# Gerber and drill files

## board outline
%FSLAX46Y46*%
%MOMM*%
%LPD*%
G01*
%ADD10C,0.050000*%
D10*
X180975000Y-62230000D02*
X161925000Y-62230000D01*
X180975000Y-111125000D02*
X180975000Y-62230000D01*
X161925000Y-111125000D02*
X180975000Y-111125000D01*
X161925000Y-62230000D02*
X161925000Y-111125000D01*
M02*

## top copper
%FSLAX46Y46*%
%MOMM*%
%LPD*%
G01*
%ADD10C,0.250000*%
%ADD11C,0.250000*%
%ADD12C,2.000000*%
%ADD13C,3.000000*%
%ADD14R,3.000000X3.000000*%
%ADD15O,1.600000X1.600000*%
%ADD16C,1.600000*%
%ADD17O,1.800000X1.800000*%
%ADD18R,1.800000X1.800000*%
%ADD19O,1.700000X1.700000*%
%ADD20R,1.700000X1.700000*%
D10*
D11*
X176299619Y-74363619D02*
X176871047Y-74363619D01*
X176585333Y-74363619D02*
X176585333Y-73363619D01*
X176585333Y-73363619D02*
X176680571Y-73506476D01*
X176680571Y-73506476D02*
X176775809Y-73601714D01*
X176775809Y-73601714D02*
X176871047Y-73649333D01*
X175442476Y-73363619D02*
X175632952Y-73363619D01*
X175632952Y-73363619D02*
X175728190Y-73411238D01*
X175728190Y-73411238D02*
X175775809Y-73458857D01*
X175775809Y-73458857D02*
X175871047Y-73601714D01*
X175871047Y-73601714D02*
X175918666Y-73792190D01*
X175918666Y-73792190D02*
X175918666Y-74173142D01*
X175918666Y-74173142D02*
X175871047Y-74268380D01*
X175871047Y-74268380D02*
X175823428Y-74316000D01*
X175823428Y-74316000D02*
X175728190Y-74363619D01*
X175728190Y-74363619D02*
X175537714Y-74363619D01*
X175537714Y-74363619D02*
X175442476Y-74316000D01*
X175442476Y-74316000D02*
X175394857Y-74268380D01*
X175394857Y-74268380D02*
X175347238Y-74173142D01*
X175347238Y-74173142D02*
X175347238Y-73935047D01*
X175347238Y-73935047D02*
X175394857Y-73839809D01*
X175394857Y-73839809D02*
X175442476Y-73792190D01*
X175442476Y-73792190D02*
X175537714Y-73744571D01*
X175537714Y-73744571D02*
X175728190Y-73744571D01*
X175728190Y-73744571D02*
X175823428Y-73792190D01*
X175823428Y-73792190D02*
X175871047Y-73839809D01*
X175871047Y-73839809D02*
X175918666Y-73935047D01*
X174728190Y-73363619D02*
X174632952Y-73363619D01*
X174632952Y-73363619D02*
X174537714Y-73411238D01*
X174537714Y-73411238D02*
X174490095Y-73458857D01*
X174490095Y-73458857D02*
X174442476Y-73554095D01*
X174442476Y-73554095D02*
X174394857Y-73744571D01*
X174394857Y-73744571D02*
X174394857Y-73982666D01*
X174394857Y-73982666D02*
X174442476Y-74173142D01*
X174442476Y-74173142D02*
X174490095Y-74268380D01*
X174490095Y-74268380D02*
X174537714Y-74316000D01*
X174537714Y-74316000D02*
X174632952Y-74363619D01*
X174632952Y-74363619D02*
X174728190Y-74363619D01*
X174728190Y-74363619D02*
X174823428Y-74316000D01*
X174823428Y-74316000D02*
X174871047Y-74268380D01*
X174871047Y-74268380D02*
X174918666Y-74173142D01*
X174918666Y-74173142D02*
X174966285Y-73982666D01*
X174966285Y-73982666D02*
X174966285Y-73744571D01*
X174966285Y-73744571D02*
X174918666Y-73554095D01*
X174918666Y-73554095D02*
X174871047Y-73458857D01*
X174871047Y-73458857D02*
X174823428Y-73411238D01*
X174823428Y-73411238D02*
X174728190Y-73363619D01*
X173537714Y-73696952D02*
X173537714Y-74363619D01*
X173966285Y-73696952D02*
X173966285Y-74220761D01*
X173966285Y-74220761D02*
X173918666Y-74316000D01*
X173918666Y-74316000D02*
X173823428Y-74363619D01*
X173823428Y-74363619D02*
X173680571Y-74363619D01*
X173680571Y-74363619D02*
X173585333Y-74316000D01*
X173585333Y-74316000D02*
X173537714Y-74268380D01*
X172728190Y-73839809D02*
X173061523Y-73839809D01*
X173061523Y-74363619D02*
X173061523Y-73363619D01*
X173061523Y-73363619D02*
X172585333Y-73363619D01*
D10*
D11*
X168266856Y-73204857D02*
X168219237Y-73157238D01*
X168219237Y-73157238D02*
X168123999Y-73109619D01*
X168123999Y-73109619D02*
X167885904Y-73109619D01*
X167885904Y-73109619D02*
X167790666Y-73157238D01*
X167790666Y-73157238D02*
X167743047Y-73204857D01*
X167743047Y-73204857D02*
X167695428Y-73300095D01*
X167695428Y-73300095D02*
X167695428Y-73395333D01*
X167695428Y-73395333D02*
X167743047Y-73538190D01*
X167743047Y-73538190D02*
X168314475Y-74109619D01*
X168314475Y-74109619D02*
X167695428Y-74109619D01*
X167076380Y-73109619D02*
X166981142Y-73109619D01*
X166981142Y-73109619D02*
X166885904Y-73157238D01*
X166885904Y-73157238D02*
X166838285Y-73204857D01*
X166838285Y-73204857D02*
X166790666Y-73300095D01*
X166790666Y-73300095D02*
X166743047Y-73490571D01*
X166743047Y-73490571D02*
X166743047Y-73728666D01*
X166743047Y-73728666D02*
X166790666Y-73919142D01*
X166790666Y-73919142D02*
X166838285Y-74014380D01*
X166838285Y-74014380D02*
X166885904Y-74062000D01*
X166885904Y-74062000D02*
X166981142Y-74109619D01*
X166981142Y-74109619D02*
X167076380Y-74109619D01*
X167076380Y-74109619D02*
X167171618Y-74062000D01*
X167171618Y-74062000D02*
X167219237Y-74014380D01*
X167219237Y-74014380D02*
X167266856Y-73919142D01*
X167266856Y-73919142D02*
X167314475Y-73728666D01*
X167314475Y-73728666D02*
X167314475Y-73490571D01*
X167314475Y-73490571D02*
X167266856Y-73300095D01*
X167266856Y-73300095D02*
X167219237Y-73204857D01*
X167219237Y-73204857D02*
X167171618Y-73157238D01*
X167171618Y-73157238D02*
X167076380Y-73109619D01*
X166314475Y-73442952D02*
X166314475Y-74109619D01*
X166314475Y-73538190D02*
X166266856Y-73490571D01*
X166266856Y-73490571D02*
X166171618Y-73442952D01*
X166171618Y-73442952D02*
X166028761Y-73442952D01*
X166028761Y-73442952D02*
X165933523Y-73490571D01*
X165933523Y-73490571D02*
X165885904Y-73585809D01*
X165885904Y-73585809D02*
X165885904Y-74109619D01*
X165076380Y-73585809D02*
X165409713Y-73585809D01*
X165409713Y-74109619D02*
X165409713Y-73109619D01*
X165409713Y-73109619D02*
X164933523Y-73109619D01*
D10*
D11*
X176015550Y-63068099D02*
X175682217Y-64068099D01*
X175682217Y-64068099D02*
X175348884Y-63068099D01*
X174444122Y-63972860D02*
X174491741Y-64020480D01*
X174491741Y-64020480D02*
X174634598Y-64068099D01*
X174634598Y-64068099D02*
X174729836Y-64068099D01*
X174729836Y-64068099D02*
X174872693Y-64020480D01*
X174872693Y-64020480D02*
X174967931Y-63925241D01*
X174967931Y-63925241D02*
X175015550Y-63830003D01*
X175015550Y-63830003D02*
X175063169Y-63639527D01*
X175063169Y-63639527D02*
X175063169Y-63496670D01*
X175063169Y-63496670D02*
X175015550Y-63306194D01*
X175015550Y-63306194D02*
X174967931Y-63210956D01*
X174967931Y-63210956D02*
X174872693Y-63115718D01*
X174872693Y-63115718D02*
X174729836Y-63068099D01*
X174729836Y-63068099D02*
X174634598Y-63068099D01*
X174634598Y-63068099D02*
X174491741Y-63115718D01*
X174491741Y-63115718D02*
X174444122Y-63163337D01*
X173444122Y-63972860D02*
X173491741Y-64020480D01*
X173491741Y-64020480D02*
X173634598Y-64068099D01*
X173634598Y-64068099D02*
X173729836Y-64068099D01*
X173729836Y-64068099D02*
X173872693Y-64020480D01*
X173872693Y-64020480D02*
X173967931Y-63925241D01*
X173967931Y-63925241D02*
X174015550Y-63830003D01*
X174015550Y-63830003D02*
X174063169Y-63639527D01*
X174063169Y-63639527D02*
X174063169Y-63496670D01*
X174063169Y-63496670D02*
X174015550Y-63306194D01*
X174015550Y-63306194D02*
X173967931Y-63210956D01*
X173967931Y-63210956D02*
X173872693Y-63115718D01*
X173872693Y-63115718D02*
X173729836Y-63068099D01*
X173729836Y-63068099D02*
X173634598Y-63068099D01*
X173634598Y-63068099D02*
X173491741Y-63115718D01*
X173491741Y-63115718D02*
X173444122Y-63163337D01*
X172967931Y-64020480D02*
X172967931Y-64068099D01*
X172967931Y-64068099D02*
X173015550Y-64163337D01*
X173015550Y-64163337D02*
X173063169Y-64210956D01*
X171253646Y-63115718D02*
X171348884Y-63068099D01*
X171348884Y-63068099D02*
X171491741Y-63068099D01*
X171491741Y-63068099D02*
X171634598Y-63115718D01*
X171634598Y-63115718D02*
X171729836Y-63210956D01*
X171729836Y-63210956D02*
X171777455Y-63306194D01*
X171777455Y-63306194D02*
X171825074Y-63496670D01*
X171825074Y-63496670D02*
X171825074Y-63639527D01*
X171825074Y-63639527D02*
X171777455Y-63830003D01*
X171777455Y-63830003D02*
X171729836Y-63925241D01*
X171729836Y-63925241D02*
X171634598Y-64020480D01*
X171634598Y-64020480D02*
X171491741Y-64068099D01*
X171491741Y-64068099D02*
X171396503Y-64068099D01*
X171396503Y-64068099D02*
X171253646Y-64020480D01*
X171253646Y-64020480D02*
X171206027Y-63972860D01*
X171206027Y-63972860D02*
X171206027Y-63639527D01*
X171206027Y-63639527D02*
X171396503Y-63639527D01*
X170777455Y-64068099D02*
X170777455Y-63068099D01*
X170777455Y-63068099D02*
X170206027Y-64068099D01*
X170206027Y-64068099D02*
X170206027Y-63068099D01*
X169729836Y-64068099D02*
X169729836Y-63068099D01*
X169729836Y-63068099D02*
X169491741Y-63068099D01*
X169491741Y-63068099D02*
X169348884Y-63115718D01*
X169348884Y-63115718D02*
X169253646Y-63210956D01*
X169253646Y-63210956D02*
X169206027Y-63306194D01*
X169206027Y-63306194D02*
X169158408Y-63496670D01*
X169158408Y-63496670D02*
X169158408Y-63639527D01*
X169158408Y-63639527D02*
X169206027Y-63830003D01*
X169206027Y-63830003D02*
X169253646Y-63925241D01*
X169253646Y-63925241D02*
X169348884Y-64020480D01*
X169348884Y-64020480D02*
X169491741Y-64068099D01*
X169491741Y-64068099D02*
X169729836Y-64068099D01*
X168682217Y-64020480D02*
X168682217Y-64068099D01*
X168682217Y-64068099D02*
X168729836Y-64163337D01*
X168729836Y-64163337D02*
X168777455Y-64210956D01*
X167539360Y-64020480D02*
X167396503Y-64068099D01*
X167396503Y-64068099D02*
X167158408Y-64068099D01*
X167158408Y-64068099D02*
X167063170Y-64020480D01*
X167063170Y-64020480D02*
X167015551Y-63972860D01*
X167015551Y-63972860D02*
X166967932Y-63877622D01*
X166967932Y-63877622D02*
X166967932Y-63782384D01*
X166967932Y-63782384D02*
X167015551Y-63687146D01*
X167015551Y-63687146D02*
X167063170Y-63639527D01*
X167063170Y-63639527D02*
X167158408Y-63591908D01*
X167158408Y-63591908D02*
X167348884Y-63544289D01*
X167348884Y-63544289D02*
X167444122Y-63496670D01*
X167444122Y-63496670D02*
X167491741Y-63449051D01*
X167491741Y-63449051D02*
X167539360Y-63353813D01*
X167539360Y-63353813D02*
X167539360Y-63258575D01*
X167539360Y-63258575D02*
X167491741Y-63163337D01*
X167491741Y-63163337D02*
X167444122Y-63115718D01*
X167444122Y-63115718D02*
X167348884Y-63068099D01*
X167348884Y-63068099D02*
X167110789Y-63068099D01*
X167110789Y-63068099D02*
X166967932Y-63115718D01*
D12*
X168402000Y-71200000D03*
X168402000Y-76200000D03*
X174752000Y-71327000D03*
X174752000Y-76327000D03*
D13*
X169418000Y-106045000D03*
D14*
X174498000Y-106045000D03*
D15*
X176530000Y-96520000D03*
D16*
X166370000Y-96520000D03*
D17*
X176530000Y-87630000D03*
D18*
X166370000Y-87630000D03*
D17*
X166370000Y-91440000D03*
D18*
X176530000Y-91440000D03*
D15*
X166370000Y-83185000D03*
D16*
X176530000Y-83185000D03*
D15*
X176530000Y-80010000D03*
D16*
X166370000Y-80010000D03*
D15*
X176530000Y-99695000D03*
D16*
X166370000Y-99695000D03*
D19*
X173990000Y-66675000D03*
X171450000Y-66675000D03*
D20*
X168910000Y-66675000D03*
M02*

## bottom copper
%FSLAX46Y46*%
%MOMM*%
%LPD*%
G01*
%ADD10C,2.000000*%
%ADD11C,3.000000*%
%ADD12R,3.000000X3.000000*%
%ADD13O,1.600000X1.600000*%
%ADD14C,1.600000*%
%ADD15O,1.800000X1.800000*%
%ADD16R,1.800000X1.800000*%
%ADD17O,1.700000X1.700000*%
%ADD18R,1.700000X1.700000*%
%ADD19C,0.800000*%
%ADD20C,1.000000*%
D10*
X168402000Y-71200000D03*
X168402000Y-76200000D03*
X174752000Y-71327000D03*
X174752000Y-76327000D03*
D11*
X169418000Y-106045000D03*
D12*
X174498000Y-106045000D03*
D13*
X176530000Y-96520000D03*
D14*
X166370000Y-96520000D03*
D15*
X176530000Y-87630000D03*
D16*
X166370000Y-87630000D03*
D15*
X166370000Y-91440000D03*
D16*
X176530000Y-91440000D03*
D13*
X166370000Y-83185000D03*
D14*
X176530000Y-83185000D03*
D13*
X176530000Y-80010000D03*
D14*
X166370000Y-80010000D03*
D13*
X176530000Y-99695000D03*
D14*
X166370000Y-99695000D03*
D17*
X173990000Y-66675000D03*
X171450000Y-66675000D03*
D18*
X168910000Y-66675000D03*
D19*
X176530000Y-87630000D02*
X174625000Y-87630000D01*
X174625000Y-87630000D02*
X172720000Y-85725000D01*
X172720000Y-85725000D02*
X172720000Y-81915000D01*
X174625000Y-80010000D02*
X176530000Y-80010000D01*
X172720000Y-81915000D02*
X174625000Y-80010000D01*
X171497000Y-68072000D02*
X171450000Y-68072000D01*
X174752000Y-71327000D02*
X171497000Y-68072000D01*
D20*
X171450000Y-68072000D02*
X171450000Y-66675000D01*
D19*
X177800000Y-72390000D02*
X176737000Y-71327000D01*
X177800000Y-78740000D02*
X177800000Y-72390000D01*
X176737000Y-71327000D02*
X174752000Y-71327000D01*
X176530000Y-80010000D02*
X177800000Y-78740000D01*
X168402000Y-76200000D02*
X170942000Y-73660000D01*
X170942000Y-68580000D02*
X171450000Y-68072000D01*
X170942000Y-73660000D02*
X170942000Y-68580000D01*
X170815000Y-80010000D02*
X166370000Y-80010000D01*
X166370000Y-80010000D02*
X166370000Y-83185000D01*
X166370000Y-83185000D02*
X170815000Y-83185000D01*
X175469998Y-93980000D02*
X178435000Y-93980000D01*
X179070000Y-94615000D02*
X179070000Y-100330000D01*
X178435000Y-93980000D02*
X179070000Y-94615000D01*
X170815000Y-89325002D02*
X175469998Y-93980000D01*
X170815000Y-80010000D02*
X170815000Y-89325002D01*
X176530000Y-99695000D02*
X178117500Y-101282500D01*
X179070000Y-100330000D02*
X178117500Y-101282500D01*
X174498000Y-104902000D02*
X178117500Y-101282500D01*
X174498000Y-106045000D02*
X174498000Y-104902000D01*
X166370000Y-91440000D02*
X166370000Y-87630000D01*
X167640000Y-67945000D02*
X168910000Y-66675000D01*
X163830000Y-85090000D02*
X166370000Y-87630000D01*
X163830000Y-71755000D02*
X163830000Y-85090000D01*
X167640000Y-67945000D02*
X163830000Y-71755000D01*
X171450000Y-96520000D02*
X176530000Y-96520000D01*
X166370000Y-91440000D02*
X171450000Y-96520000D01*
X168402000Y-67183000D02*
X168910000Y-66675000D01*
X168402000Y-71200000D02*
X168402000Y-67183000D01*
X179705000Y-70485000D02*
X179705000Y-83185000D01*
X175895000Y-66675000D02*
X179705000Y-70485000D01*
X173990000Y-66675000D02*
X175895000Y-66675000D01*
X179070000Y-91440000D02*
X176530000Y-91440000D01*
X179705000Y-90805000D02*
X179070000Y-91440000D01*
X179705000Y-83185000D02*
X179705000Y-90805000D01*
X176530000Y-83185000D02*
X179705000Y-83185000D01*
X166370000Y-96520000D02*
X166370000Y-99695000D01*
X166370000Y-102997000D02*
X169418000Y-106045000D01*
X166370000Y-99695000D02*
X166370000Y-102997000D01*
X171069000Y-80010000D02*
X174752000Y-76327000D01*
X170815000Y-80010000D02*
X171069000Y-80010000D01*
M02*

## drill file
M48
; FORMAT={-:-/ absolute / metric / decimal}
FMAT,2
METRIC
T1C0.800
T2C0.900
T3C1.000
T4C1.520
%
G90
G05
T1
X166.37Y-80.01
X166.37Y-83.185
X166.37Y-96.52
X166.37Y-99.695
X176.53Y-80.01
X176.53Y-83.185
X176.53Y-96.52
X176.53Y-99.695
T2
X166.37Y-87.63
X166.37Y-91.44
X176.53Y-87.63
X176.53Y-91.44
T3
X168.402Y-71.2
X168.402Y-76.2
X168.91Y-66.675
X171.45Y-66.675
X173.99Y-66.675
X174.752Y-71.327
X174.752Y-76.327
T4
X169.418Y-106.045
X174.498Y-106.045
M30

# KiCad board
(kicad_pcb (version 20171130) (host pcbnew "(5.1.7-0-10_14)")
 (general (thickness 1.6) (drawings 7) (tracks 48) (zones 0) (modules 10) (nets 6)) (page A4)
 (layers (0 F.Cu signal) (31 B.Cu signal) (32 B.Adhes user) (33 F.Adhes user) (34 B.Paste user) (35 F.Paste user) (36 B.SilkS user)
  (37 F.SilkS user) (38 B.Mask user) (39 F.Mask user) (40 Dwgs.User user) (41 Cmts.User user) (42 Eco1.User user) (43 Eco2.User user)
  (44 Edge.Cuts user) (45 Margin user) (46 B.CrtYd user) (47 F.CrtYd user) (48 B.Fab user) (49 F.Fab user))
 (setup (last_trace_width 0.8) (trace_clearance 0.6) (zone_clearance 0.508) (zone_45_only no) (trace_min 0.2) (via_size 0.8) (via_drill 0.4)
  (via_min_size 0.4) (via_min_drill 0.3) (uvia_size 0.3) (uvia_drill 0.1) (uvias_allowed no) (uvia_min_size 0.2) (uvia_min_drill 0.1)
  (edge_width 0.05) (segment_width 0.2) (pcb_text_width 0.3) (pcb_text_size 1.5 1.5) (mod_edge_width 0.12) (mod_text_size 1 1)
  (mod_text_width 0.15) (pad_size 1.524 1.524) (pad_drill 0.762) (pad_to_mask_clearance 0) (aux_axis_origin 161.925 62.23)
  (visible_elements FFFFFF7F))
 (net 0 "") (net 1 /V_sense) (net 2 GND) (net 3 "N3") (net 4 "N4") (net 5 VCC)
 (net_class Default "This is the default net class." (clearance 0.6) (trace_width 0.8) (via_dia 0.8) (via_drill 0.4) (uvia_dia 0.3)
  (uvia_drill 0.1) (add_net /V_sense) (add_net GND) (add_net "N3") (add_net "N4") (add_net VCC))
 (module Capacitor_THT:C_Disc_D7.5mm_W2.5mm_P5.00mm (layer F.Cu) (at 168.402 76.2 90)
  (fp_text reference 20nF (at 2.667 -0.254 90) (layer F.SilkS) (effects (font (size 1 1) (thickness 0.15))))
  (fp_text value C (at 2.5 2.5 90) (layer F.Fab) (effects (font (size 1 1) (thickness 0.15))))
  (pad 2 thru_hole circle (at 5 0 90) (size 2 2) (drill 1) (layers *.Cu *.Mask) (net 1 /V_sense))
  (pad 1 thru_hole circle (at 0 0 90) (size 2 2) (drill 1) (layers *.Cu *.Mask) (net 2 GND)))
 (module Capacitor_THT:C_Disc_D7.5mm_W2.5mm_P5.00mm (layer F.Cu) (at 174.752 76.327 90)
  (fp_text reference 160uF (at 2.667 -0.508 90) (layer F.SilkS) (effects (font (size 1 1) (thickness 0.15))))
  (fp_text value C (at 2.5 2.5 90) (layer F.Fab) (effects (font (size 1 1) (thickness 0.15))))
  (pad 2 thru_hole circle (at 5 0 90) (size 2 2) (drill 1) (layers *.Cu *.Mask) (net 2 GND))
  (pad 1 thru_hole circle (at 0 0 90) (size 2 2) (drill 1) (layers *.Cu *.Mask) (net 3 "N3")))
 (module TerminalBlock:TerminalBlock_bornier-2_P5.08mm (layer F.Cu) (at 174.498 106.045 180)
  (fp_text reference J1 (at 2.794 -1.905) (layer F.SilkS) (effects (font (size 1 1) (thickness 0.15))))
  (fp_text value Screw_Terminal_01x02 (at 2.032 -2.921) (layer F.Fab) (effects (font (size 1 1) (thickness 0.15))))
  (pad 2 thru_hole circle (at 5.08 0 180) (size 3 3) (drill 1.52) (layers *.Cu *.Mask) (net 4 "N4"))
  (pad 1 thru_hole rect (at 0 0 180) (size 3 3) (drill 1.52) (layers *.Cu *.Mask) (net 3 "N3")))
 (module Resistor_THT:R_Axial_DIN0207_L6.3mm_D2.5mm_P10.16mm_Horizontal (layer F.Cu) (at 166.37 96.52)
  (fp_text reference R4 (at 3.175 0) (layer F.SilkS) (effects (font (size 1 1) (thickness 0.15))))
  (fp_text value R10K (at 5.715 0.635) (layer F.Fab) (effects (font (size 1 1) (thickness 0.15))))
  (pad 2 thru_hole oval (at 10.16 0) (size 1.6 1.6) (drill 0.8) (layers *.Cu *.Mask) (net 1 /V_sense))
  (pad 1 thru_hole circle (at 0 0) (size 1.6 1.6) (drill 0.8) (layers *.Cu *.Mask) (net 4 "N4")))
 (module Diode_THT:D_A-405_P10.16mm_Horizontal (layer F.Cu) (at 166.37 87.63)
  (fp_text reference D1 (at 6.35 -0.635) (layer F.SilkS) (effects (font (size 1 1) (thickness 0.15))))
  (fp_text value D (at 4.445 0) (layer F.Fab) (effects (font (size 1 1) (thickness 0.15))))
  (pad 2 thru_hole oval (at 10.16 0) (size 1.8 1.8) (drill 0.9) (layers *.Cu *.Mask) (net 2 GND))
  (pad 1 thru_hole rect (at 0 0) (size 1.8 1.8) (drill 0.9) (layers *.Cu *.Mask) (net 1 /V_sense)))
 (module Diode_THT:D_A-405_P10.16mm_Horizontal (layer F.Cu) (at 176.53 91.44 180)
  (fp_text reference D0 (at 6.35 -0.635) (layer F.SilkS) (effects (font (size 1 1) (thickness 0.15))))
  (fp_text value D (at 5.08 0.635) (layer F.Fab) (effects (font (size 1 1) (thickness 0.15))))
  (pad 2 thru_hole oval (at 10.16 0 180) (size 1.8 1.8) (drill 0.9) (layers *.Cu *.Mask) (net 1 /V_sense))
  (pad 1 thru_hole rect (at 0 0 180) (size 1.8 1.8) (drill 0.9) (layers *.Cu *.Mask) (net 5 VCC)))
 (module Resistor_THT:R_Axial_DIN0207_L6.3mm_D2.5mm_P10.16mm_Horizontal (layer F.Cu) (at 176.53 83.185 180)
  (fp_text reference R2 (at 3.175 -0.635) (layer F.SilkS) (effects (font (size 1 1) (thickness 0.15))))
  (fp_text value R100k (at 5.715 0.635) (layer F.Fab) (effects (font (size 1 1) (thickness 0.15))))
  (pad 2 thru_hole oval (at 10.16 0 180) (size 1.6 1.6) (drill 0.8) (layers *.Cu *.Mask) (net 3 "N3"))
  (pad 1 thru_hole circle (at 0 0 180) (size 1.6 1.6) (drill 0.8) (layers *.Cu *.Mask) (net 5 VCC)))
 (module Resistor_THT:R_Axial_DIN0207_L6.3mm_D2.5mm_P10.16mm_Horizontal (layer F.Cu) (at 166.37 80.01)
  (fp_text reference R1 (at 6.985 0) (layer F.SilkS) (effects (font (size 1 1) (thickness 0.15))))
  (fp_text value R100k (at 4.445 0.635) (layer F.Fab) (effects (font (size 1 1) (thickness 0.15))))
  (pad 2 thru_hole oval (at 10.16 0) (size 1.6 1.6) (drill 0.8) (layers *.Cu *.Mask) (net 2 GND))
  (pad 1 thru_hole circle (at 0 0) (size 1.6 1.6) (drill 0.8) (layers *.Cu *.Mask) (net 3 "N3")))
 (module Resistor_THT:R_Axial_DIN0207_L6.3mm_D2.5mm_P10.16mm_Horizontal (layer F.Cu) (at 166.37 99.695)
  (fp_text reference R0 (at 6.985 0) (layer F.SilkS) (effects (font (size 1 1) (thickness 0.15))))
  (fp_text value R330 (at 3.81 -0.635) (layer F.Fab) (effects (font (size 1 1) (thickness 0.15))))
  (pad 2 thru_hole oval (at 10.16 0) (size 1.6 1.6) (drill 0.8) (layers *.Cu *.Mask) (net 3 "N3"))
  (pad 1 thru_hole circle (at 0 0) (size 1.6 1.6) (drill 0.8) (layers *.Cu *.Mask) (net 4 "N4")))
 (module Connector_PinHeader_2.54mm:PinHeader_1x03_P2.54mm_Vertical (layer F.Cu) (at 168.91 66.675 90)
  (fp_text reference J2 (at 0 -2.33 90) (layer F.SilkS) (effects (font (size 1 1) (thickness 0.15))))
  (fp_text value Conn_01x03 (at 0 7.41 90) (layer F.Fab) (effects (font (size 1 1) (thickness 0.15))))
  (pad 3 thru_hole oval (at 0 5.08 90) (size 1.7 1.7) (drill 1) (layers *.Cu *.Mask) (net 5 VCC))
  (pad 2 thru_hole oval (at 0 2.54 90) (size 1.7 1.7) (drill 1) (layers *.Cu *.Mask) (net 2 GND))
  (pad 1 thru_hole rect (at 0 0 90) (size 1.7 1.7) (drill 1) (layers *.Cu *.Mask) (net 1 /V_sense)))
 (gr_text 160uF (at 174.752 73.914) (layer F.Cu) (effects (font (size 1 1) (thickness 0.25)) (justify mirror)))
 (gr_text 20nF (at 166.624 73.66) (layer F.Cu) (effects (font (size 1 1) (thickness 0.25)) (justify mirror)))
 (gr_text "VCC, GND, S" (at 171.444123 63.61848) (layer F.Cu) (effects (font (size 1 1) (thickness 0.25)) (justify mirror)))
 (gr_line (start 180.975 62.23) (end 161.925 62.23) (layer Edge.Cuts) (width 0.05))
 (gr_line (start 180.975 111.125) (end 180.975 62.23) (layer Edge.Cuts) (width 0.05))
 (gr_line (start 161.925 111.125) (end 180.975 111.125) (layer Edge.Cuts) (width 0.05))
 (gr_line (start 161.925 62.23) (end 161.925 111.125) (layer Edge.Cuts) (width 0.05))
 (segment (start 176.53 87.63) (end 174.625 87.63) (width 0.8) (layer B.Cu) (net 2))
 (segment (start 174.625 87.63) (end 172.72 85.725) (width 0.8) (layer B.Cu) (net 2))
 (segment (start 172.72 85.725) (end 172.72 81.915) (width 0.8) (layer B.Cu) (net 2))
 (segment (start 174.625 80.01) (end 176.53 80.01) (width 0.8) (layer B.Cu) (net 2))
 (segment (start 172.72 81.915) (end 174.625 80.01) (width 0.8) (layer B.Cu) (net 2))
 (segment (start 171.497 68.072) (end 171.45 68.072) (width 0.8) (layer B.Cu) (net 2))
 (segment (start 174.752 71.327) (end 171.497 68.072) (width 0.8) (layer B.Cu) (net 2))
 (segment (start 171.45 68.072) (end 171.45 66.675) (width 1) (layer B.Cu) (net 2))
 (segment (start 177.8 72.39) (end 176.737 71.327) (width 0.8) (layer B.Cu) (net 2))
 (segment (start 177.8 78.74) (end 177.8 72.39) (width 0.8) (layer B.Cu) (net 2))
 (segment (start 176.737 71.327) (end 174.752 71.327) (width 0.8) (layer B.Cu) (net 2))
 (segment (start 176.53 80.01) (end 177.8 78.74) (width 0.8) (layer B.Cu) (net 2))
 (segment (start 168.402 76.2) (end 170.942 73.66) (width 0.8) (layer B.Cu) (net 2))
 (segment (start 170.942 68.58) (end 171.45 68.072) (width 0.8) (layer B.Cu) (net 2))
 (segment (start 170.942 73.66) (end 170.942 68.58) (width 0.8) (layer B.Cu) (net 2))
 (segment (start 170.815 80.01) (end 166.37 80.01) (width 0.8) (layer B.Cu) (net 3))
 (segment (start 166.37 80.01) (end 166.37 83.185) (width 0.8) (layer B.Cu) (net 3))
 (segment (start 166.37 83.185) (end 170.815 83.185) (width 0.8) (layer B.Cu) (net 3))
 (segment (start 175.469998 93.98) (end 178.435 93.98) (width 0.8) (layer B.Cu) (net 3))
 (segment (start 179.07 94.615) (end 179.07 100.33) (width 0.8) (layer B.Cu) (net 3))
 (segment (start 178.435 93.98) (end 179.07 94.615) (width 0.8) (layer B.Cu) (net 3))
 (segment (start 170.815 89.325002) (end 175.469998 93.98) (width 0.8) (layer B.Cu) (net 3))
 (segment (start 170.815 80.01) (end 170.815 89.325002) (width 0.8) (layer B.Cu) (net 3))
 (segment (start 176.53 99.695) (end 178.1175 101.2825) (width 0.8) (layer B.Cu) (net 3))
 (segment (start 179.07 100.33) (end 178.1175 101.2825) (width 0.8) (layer B.Cu) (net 3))
 (segment (start 174.498 104.902) (end 178.1175 101.2825) (width 0.8) (layer B.Cu) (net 3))
 (segment (start 174.498 106.045) (end 174.498 104.902) (width 0.8) (layer B.Cu) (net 3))
 (segment (start 166.37 91.44) (end 166.37 87.63) (width 0.8) (layer B.Cu) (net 1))
 (segment (start 167.64 67.945) (end 168.91 66.675) (width 0.8) (layer B.Cu) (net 1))
 (segment (start 163.83 85.09) (end 166.37 87.63) (width 0.8) (layer B.Cu) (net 1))
 (segment (start 163.83 71.755) (end 163.83 85.09) (width 0.8) (layer B.Cu) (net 1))
 (segment (start 167.64 67.945) (end 163.83 71.755) (width 0.8) (layer B.Cu) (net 1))
 (segment (start 171.45 96.52) (end 176.53 96.52) (width 0.8) (layer B.Cu) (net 1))
 (segment (start 166.37 91.44) (end 171.45 96.52) (width 0.8) (layer B.Cu) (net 1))
 (segment (start 168.402 67.183) (end 168.91 66.675) (width 0.8) (layer B.Cu) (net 1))
 (segment (start 168.402 71.2) (end 168.402 67.183) (width 0.8) (layer B.Cu) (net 1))
 (segment (start 179.705 70.485) (end 179.705 83.185) (width 0.8) (layer B.Cu) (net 5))
 (segment (start 175.895 66.675) (end 179.705 70.485) (width 0.8) (layer B.Cu) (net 5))
 (segment (start 173.99 66.675) (end 175.895 66.675) (width 0.8) (layer B.Cu) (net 5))
 (segment (start 179.07 91.44) (end 176.53 91.44) (width 0.8) (layer B.Cu) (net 5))
 (segment (start 179.705 90.805) (end 179.07 91.44) (width 0.8) (layer B.Cu) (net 5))
 (segment (start 179.705 83.185) (end 179.705 90.805) (width 0.8) (layer B.Cu) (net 5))
 (segment (start 176.53 83.185) (end 179.705 83.185) (width 0.8) (layer B.Cu) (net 5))
 (segment (start 166.37 96.52) (end 166.37 99.695) (width 0.8) (layer B.Cu) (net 4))
 (segment (start 166.37 102.997) (end 169.418 106.045) (width 0.8) (layer B.Cu) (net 4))
 (segment (start 166.37 99.695) (end 166.37 102.997) (width 0.8) (layer B.Cu) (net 4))
 (segment (start 171.069 80.01) (end 174.752 76.327) (width 0.8) (layer B.Cu) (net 3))
 (segment (start 170.815 80.01) (end 171.069 80.01) (width 0.8) (layer B.Cu) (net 3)))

